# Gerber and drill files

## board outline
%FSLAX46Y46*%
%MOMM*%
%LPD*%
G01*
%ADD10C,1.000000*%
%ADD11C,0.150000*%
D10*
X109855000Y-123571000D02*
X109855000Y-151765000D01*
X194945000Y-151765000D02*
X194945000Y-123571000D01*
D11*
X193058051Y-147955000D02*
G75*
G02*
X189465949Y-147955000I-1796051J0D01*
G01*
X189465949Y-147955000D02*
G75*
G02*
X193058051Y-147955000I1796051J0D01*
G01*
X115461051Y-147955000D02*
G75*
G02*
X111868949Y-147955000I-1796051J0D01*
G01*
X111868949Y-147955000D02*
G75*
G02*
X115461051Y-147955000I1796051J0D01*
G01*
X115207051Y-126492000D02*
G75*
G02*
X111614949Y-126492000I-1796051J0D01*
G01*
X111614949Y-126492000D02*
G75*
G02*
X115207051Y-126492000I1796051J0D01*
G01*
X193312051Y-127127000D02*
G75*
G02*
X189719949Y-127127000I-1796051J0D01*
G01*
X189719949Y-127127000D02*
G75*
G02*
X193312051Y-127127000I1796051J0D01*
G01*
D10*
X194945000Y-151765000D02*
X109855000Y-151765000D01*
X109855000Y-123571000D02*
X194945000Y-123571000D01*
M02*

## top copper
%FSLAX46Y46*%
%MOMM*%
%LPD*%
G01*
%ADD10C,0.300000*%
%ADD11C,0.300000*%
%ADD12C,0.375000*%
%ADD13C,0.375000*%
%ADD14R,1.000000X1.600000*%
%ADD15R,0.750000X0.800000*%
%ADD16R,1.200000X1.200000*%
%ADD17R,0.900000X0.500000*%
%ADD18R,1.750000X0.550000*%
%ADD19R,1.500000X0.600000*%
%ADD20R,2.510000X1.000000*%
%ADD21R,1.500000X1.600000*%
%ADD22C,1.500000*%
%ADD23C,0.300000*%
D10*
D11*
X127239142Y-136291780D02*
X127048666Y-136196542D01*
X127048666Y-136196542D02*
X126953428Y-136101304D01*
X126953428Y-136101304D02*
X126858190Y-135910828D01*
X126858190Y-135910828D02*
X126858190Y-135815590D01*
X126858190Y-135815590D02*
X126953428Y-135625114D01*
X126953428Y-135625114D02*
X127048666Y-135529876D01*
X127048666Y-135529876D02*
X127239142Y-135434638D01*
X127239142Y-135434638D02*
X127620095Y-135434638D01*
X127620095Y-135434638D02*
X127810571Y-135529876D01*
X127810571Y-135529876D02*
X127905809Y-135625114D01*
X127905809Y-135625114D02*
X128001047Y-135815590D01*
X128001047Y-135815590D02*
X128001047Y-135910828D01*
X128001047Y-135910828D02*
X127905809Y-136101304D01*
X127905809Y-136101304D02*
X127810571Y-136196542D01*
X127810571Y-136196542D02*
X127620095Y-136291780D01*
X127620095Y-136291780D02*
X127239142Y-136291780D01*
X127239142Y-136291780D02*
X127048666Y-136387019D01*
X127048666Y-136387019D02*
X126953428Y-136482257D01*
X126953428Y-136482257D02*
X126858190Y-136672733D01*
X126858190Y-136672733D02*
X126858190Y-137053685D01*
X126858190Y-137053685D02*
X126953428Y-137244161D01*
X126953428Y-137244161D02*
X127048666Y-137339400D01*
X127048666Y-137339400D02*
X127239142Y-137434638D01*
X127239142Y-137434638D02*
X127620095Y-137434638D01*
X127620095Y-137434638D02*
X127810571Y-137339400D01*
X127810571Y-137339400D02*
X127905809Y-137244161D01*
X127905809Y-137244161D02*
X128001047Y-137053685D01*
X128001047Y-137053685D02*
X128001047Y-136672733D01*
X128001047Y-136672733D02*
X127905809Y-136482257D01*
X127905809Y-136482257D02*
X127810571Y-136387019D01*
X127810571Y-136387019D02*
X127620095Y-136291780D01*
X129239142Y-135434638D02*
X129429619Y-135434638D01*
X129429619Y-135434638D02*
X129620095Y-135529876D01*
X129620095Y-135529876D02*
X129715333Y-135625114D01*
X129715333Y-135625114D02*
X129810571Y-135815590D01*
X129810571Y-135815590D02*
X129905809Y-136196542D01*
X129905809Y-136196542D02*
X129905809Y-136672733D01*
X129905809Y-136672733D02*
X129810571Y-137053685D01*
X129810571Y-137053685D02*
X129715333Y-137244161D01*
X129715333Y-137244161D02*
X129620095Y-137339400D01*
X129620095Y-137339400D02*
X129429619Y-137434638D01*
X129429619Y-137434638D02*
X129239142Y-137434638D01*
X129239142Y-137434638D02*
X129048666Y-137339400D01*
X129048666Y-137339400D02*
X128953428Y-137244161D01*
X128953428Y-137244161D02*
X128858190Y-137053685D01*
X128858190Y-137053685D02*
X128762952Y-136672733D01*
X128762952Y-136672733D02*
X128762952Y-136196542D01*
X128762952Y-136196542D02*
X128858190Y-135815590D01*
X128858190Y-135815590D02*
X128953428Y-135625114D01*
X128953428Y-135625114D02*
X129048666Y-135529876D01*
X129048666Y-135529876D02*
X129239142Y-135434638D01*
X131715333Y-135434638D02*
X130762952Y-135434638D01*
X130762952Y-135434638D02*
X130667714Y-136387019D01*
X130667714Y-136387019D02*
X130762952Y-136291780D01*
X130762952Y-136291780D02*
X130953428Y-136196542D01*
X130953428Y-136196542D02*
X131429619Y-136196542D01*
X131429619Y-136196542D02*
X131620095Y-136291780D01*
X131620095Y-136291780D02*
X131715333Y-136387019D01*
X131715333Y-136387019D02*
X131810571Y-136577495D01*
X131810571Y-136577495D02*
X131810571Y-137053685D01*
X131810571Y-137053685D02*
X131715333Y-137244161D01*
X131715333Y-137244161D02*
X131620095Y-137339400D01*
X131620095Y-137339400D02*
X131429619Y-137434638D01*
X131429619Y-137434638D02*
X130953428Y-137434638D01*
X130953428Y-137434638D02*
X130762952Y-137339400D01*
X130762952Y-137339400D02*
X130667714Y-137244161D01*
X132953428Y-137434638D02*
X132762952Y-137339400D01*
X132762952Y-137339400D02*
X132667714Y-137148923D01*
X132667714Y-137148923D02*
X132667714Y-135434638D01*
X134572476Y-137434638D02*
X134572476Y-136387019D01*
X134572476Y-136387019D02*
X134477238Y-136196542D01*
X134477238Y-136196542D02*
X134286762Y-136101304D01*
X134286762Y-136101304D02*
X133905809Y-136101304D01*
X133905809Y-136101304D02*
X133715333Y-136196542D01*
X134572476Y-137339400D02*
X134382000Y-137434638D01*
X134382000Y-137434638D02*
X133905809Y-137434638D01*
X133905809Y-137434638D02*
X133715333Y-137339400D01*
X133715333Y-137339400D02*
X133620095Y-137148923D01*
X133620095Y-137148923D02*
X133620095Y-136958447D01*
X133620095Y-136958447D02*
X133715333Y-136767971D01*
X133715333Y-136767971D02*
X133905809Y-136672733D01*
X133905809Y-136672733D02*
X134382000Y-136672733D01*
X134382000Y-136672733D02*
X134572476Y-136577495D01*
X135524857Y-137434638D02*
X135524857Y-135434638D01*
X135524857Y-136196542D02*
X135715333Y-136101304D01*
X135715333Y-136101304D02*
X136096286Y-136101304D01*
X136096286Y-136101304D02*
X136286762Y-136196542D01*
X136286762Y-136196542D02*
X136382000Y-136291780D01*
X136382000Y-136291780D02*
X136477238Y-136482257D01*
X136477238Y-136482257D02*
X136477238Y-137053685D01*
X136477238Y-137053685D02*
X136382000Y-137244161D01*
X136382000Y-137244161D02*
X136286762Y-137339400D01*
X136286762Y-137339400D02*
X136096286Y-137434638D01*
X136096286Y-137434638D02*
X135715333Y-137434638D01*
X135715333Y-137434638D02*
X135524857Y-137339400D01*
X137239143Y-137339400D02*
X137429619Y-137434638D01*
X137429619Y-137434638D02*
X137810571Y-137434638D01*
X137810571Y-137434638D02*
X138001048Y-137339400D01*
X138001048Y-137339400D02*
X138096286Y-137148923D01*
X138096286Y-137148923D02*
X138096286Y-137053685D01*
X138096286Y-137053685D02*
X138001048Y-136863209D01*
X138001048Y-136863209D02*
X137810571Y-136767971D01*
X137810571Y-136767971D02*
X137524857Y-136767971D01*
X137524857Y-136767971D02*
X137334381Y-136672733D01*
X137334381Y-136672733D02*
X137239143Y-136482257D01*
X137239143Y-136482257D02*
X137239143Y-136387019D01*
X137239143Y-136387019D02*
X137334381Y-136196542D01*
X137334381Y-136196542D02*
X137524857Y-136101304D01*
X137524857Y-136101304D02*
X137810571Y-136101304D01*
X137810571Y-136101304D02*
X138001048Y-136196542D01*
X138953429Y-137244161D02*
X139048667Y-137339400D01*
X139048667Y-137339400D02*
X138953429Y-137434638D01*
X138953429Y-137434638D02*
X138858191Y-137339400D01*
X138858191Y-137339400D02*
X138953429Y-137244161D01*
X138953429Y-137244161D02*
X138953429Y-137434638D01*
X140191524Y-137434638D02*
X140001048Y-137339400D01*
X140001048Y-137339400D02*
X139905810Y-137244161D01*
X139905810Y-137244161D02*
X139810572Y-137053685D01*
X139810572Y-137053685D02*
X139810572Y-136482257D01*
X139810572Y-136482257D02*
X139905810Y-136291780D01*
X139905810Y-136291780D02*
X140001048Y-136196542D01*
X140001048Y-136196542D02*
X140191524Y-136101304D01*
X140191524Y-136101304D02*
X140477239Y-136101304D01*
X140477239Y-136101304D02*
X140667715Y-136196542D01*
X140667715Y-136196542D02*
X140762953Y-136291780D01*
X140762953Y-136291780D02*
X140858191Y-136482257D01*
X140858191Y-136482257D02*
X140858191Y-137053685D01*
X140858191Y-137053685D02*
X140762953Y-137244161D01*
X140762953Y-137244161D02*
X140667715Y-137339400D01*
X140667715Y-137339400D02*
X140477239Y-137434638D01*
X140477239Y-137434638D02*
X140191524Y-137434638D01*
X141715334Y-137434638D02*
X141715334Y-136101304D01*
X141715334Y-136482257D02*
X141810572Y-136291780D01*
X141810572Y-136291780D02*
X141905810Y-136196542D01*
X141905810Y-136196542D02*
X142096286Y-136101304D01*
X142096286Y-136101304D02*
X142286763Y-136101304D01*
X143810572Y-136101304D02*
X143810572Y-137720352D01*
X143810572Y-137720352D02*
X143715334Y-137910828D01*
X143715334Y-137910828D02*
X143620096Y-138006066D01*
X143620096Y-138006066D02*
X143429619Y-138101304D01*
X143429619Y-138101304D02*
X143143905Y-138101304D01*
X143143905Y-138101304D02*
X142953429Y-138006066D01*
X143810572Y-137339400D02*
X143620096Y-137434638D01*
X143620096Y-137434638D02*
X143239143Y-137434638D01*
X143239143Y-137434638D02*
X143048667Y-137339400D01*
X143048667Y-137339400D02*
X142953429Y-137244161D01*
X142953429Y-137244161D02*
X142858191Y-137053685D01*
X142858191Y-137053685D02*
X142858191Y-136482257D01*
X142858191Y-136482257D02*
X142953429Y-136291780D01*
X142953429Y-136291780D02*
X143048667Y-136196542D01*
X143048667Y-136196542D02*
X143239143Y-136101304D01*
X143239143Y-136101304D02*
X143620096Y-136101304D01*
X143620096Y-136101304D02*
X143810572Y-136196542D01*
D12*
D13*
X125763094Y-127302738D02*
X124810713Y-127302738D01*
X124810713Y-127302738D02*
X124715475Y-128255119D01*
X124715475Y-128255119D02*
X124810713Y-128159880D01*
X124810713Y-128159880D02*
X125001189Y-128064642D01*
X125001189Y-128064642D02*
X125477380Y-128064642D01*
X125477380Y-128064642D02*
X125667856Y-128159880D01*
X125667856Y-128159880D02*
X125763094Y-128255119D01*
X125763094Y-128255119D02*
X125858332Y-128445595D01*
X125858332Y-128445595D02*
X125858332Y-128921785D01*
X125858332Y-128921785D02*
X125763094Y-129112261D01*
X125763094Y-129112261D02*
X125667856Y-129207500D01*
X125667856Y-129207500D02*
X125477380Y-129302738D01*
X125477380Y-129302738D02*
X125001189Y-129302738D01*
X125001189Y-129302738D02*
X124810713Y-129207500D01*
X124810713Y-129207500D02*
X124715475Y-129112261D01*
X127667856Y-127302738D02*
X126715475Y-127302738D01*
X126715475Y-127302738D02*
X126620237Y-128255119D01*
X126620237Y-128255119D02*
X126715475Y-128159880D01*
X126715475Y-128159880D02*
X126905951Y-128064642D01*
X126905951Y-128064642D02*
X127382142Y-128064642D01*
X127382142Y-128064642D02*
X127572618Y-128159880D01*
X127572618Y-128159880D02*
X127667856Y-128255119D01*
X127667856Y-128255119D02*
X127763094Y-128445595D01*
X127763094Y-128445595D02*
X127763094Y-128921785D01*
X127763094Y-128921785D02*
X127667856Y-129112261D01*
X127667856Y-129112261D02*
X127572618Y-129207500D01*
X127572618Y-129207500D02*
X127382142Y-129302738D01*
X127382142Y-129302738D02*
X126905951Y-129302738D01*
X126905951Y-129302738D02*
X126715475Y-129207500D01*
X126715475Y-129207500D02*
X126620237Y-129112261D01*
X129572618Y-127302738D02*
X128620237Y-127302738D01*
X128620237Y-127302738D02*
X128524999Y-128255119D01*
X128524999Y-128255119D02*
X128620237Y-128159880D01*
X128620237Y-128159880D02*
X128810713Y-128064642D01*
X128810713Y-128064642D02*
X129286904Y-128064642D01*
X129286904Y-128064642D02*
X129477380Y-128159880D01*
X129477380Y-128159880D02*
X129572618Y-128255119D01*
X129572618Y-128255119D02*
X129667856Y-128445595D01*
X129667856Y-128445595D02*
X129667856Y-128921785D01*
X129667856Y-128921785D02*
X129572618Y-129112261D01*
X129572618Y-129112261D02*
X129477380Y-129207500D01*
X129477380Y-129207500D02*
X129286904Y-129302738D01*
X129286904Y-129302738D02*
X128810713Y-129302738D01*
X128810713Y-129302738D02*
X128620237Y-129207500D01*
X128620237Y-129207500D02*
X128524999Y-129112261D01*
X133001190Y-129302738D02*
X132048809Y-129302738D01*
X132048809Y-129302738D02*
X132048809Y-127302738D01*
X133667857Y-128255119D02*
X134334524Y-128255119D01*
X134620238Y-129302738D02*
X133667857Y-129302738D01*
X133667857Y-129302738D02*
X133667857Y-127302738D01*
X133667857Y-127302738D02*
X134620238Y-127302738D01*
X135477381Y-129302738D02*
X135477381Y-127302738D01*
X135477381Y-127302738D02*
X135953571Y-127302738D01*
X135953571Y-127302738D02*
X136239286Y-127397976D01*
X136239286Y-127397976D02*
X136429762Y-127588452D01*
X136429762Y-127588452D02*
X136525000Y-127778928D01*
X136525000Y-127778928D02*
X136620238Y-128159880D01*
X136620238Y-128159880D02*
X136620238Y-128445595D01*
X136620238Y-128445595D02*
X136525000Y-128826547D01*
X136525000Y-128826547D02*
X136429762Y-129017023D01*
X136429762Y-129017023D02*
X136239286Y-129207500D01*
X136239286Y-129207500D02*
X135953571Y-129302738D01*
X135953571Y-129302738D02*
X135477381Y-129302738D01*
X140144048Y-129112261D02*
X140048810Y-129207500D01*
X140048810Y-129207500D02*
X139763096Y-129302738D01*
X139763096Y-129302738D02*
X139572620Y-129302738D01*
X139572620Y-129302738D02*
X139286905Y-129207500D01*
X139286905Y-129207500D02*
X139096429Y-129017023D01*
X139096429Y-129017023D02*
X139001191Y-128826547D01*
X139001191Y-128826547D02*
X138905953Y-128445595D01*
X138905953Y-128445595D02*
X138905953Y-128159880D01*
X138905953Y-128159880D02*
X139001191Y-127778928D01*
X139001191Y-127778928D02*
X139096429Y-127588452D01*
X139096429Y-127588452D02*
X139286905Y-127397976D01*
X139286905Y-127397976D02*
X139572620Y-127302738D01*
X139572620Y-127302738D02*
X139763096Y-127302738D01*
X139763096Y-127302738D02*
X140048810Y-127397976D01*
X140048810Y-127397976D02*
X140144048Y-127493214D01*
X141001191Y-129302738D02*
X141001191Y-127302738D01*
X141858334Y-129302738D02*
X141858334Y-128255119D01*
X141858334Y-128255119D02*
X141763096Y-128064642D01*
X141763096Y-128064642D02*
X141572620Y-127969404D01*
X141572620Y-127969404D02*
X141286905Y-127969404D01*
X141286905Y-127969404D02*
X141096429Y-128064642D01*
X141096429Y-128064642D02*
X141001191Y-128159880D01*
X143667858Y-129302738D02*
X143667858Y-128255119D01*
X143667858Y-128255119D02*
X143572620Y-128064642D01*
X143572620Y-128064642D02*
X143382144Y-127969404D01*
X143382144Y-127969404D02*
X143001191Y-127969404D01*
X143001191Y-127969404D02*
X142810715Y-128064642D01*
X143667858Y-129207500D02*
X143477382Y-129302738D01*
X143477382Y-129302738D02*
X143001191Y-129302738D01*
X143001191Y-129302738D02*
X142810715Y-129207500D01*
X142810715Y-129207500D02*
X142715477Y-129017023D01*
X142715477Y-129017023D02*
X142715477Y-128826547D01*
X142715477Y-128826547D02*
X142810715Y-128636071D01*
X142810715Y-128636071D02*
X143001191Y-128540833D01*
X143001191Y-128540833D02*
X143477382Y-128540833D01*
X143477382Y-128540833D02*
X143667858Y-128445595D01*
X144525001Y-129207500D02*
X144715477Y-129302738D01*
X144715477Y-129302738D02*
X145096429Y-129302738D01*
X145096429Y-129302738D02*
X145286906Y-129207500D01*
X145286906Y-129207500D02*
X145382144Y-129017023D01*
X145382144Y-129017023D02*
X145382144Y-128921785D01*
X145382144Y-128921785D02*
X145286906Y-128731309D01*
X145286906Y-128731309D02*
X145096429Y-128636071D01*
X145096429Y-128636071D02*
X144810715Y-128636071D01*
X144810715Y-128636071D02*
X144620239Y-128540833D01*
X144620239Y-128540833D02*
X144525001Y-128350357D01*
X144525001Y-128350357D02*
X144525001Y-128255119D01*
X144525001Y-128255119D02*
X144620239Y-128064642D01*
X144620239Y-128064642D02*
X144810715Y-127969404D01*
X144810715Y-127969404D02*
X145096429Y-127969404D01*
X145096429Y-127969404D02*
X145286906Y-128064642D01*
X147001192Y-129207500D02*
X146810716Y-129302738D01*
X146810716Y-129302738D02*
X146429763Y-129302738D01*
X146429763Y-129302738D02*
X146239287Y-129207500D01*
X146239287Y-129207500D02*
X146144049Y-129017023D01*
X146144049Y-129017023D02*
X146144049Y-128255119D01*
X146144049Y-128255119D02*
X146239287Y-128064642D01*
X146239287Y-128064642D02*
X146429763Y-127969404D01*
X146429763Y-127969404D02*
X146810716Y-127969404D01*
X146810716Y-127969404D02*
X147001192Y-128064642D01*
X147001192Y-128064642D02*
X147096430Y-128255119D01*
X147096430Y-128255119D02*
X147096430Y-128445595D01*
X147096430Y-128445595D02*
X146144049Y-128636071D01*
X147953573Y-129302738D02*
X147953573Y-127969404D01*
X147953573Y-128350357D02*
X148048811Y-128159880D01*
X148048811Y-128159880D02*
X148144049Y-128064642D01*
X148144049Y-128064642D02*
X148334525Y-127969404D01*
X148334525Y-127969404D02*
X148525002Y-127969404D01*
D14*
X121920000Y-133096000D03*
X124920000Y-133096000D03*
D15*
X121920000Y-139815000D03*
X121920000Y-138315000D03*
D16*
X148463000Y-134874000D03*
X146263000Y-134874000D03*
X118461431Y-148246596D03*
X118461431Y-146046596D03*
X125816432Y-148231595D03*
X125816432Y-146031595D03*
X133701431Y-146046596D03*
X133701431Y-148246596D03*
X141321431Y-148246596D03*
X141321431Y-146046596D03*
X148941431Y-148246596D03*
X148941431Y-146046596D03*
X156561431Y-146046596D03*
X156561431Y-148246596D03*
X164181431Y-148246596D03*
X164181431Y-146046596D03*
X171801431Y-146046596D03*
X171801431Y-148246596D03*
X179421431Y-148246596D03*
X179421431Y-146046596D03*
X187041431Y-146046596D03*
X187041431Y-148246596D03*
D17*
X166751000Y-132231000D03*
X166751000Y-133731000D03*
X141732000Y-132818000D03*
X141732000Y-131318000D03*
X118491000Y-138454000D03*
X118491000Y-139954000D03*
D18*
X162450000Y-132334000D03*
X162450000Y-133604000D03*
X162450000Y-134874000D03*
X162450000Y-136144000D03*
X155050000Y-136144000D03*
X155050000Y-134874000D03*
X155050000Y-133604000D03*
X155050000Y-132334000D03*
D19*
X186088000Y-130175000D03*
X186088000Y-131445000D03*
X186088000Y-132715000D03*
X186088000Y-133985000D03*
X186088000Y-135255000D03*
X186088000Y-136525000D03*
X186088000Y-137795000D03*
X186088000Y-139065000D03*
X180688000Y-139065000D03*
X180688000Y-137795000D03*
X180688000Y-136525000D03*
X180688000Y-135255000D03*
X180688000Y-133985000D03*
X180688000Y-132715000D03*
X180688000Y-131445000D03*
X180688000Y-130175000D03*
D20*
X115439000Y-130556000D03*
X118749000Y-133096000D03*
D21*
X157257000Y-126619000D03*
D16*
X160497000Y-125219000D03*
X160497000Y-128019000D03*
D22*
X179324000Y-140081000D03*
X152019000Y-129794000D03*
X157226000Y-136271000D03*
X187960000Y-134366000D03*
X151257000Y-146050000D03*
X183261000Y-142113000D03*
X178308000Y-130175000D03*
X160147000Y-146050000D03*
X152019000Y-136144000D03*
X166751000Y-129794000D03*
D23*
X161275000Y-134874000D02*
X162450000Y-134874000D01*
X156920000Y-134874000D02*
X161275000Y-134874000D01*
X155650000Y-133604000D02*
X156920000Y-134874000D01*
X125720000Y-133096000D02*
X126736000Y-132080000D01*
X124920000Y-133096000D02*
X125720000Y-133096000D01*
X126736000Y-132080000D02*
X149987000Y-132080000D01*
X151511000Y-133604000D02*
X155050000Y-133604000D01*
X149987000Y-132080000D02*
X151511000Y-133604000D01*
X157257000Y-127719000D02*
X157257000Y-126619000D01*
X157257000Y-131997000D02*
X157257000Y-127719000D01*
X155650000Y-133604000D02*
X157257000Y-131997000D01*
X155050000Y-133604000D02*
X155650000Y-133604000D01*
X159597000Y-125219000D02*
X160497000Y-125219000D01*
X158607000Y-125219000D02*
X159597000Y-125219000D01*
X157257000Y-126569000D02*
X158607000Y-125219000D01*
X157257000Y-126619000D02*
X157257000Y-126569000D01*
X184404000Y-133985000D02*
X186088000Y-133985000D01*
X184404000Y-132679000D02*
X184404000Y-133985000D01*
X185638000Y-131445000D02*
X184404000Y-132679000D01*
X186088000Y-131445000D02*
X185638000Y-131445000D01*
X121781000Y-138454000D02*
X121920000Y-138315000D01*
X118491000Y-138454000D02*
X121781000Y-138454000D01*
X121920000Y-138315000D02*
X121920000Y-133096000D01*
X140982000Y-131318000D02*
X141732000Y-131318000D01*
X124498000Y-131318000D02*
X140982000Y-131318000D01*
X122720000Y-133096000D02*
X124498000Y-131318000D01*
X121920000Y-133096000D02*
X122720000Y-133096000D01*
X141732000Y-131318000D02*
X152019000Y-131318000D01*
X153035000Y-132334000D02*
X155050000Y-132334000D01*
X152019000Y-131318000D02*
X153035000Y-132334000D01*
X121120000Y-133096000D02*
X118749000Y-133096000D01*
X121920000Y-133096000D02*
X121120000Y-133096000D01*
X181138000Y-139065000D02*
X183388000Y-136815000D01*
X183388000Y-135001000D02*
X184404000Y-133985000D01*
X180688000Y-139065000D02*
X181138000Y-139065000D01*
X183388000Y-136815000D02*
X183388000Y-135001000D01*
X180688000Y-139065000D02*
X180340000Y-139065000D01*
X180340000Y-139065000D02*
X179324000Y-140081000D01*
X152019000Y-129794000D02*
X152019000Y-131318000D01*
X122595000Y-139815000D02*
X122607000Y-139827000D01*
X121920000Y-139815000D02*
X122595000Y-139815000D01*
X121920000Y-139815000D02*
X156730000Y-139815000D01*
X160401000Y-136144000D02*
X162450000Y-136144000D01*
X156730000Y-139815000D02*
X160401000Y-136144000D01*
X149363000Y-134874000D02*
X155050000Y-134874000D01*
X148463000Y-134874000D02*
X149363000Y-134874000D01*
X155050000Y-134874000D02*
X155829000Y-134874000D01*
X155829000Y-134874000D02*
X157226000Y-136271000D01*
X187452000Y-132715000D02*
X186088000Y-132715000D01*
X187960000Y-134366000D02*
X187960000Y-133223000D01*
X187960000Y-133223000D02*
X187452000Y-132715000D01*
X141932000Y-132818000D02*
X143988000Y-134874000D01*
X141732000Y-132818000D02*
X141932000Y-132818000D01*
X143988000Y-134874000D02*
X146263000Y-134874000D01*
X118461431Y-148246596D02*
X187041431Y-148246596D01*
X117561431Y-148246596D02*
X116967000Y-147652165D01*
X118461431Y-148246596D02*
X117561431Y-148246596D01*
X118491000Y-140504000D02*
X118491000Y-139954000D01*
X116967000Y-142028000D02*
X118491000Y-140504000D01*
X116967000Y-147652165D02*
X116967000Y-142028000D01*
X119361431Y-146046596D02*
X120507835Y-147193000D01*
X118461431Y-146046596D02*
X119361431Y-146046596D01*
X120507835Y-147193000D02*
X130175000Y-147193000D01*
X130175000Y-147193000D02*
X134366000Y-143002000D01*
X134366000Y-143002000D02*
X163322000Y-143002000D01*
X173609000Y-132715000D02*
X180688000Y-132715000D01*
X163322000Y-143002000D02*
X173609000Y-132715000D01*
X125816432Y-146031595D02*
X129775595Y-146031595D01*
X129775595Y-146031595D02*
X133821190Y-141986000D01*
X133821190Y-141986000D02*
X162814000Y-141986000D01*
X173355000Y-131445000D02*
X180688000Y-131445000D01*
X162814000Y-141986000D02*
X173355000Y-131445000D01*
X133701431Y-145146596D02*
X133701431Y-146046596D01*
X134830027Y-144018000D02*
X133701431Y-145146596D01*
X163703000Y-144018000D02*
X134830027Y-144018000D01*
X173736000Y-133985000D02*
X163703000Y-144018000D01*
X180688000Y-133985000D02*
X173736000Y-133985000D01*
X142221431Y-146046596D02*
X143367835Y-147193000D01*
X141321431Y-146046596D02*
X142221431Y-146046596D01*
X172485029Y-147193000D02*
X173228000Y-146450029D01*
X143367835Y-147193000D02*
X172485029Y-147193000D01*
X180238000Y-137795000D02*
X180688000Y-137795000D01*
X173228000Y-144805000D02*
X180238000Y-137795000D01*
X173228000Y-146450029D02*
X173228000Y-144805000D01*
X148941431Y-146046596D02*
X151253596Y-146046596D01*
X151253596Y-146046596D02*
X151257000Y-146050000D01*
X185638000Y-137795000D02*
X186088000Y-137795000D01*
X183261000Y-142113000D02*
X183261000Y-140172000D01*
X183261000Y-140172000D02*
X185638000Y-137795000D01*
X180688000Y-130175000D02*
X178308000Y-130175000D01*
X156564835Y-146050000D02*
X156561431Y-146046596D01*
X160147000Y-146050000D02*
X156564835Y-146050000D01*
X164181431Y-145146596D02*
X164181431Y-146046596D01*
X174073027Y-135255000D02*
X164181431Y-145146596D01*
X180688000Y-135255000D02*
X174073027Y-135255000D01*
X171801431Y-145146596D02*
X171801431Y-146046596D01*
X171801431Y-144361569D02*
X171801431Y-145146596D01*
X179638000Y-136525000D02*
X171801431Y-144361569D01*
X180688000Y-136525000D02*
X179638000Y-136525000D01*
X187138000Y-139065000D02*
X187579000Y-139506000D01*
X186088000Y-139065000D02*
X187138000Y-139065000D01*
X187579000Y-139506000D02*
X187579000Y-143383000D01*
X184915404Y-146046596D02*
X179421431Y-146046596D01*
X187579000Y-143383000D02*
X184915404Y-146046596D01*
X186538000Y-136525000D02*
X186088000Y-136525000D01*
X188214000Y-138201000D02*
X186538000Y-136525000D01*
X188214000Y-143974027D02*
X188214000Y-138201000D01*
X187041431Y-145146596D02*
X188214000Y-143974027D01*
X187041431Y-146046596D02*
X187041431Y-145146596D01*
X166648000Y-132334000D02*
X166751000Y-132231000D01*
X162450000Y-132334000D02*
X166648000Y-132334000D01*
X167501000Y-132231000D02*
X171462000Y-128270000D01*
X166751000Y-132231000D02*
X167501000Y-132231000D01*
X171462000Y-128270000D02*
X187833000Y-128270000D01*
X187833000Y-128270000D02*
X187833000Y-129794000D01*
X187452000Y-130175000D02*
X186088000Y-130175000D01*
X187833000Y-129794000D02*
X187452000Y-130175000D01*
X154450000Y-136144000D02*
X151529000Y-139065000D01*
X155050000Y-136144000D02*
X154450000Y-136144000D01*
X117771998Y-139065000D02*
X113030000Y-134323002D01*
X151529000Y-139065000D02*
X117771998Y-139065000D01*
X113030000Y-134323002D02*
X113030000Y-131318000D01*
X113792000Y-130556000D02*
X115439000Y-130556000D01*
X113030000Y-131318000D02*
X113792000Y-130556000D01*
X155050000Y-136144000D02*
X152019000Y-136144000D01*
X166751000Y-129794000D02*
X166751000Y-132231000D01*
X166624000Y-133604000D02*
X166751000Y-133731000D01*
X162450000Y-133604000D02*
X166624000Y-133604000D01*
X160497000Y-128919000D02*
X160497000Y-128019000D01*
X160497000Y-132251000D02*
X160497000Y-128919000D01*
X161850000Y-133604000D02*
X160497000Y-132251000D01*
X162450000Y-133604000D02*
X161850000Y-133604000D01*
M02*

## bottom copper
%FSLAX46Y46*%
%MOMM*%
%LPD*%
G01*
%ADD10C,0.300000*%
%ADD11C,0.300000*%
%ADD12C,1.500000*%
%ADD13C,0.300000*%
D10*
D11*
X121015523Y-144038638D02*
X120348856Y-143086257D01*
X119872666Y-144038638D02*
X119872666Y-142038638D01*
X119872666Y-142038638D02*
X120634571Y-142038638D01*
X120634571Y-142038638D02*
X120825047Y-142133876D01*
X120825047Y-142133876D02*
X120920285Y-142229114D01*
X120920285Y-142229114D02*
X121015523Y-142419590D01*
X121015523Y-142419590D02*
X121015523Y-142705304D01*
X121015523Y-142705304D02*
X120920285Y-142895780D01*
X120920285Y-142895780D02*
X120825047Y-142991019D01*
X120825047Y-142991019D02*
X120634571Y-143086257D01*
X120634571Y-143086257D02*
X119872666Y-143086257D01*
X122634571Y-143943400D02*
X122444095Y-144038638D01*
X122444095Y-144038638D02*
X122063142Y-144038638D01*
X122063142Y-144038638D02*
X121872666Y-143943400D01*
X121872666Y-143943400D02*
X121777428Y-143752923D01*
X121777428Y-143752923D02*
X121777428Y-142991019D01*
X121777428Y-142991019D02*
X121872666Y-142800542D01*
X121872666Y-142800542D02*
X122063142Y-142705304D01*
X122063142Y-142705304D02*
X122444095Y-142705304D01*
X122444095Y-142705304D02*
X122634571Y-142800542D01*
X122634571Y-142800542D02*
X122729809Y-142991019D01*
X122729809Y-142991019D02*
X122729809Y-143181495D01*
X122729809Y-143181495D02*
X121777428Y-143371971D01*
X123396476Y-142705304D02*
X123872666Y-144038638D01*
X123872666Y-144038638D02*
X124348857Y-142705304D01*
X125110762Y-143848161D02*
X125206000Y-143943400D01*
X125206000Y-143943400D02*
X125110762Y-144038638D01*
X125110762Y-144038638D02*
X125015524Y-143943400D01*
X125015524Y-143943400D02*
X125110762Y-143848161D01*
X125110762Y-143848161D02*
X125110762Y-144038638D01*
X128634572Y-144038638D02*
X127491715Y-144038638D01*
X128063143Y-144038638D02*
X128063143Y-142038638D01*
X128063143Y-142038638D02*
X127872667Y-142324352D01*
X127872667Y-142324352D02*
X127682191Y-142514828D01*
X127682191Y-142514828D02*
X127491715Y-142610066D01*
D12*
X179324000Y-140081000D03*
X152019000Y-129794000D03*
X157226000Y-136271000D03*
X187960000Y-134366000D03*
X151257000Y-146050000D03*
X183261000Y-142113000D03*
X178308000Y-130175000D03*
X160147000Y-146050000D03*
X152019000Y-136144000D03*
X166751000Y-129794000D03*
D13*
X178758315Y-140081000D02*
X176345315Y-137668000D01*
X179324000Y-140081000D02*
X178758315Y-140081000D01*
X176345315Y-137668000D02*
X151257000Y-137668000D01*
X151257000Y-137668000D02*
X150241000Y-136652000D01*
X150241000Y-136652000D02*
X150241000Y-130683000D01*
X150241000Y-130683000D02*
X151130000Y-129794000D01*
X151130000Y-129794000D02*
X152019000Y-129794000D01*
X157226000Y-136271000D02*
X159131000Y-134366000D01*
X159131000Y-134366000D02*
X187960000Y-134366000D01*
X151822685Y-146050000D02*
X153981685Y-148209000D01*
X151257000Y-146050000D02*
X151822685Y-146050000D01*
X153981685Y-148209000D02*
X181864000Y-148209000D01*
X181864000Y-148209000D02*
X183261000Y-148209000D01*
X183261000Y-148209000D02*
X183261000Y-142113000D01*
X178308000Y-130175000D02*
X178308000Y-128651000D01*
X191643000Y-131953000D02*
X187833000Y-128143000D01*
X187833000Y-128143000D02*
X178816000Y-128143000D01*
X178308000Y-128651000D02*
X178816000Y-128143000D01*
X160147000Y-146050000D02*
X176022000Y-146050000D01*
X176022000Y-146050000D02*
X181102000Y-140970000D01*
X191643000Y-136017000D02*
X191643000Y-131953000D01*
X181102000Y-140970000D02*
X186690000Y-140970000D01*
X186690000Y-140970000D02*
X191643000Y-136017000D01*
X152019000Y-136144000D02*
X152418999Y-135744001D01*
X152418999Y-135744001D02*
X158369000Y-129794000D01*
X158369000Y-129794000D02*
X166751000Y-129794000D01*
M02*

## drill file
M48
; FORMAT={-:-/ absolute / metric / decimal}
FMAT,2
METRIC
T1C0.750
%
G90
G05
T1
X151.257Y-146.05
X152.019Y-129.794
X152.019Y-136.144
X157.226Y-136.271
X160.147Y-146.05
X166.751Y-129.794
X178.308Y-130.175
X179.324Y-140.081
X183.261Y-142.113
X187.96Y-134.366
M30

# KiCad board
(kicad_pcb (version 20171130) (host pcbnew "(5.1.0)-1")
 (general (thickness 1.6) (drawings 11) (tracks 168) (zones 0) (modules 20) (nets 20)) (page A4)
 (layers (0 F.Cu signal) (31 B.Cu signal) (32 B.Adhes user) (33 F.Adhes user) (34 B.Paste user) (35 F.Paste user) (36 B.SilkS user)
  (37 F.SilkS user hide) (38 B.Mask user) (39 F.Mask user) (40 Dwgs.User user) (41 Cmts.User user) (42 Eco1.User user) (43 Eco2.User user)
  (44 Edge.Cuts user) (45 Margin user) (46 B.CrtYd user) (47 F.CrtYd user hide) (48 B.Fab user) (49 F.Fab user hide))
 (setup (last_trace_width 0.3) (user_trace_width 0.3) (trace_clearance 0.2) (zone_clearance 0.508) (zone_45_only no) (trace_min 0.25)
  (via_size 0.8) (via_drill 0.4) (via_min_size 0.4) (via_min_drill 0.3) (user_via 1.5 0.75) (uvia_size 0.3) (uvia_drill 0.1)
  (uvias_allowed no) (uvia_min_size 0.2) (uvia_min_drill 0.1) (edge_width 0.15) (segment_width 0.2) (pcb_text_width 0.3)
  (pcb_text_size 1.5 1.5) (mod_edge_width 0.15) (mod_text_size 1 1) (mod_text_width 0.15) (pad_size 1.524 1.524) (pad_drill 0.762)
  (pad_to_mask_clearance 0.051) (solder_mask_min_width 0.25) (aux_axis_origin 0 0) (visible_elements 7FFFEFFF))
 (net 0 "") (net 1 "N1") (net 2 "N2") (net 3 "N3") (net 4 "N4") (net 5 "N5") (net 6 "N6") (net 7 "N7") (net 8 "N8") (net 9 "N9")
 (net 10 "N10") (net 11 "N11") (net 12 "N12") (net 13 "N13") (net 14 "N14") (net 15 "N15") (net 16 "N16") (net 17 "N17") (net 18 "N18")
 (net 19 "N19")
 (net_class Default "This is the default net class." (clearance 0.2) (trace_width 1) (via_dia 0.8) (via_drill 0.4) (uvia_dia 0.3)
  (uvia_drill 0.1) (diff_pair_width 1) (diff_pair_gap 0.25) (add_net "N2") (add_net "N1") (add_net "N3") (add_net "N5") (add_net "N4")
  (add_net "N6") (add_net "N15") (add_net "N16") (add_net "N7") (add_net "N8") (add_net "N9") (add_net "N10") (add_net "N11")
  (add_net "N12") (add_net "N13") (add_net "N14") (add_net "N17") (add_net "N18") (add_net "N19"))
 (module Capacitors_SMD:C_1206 (layer F.Cu) (at 123.42 133.096 180)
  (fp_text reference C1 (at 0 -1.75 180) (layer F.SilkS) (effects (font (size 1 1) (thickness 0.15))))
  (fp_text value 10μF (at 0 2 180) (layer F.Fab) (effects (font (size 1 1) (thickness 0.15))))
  (pad 2 smd rect (at 1.5 0 180) (size 1 1.6) (layers F.Cu F.Paste F.Mask) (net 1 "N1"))
  (pad 1 smd rect (at -1.5 0 180) (size 1 1.6) (layers F.Cu F.Paste F.Mask) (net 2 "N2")))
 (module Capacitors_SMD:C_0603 (layer F.Cu) (at 121.92 139.065 90)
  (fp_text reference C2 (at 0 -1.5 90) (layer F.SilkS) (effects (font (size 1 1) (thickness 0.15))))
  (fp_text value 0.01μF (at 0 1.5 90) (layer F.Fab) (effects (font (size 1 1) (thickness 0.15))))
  (pad 1 smd rect (at -0.75 0 90) (size 0.8 0.75) (layers F.Cu F.Paste F.Mask) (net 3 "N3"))
  (pad 2 smd rect (at 0.75 0 90) (size 0.8 0.75) (layers F.Cu F.Paste F.Mask) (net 1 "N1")))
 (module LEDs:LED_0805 (layer F.Cu) (at 147.363 134.874)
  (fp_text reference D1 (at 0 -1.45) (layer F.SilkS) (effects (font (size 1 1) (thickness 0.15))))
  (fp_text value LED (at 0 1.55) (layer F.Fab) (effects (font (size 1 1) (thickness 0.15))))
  (pad 2 smd rect (at 1.1 0 180) (size 1.2 1.2) (layers F.Cu F.Paste F.Mask) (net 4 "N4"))
  (pad 1 smd rect (at -1.1 0 180) (size 1.2 1.2) (layers F.Cu F.Paste F.Mask) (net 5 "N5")))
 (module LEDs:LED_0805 (layer F.Cu) (at 118.461431 147.146596 90)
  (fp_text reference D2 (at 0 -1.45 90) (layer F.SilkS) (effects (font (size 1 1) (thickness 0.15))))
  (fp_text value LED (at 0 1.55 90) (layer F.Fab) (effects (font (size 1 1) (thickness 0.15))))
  (pad 1 smd rect (at -1.1 0 270) (size 1.2 1.2) (layers F.Cu F.Paste F.Mask) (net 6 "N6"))
  (pad 2 smd rect (at 1.1 0 270) (size 1.2 1.2) (layers F.Cu F.Paste F.Mask) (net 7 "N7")))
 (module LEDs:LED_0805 (layer F.Cu) (at 125.816432 147.131595 90)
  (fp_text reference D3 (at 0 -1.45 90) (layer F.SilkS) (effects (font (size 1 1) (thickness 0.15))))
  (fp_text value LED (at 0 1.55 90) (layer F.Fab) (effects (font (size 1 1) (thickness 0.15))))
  (pad 1 smd rect (at -1.1 0 270) (size 1.2 1.2) (layers F.Cu F.Paste F.Mask) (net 6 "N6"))
  (pad 2 smd rect (at 1.1 0 270) (size 1.2 1.2) (layers F.Cu F.Paste F.Mask) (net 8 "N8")))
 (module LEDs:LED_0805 (layer F.Cu) (at 133.701431 147.146596 90)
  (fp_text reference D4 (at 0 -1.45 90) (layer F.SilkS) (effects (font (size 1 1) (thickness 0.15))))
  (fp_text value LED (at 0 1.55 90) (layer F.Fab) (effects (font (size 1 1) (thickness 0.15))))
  (pad 2 smd rect (at 1.1 0 270) (size 1.2 1.2) (layers F.Cu F.Paste F.Mask) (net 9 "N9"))
  (pad 1 smd rect (at -1.1 0 270) (size 1.2 1.2) (layers F.Cu F.Paste F.Mask) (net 6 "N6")))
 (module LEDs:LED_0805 (layer F.Cu) (at 141.321431 147.146596 90)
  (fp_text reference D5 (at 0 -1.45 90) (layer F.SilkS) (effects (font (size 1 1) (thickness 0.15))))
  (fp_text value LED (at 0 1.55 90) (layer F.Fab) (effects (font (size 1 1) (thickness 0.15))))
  (pad 1 smd rect (at -1.1 0 270) (size 1.2 1.2) (layers F.Cu F.Paste F.Mask) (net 6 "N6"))
  (pad 2 smd rect (at 1.1 0 270) (size 1.2 1.2) (layers F.Cu F.Paste F.Mask) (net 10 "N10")))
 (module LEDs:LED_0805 (layer F.Cu) (at 148.941431 147.146596 90)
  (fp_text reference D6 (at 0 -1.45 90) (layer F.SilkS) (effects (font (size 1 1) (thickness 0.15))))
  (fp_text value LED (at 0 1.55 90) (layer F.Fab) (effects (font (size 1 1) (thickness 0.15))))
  (pad 1 smd rect (at -1.1 0 270) (size 1.2 1.2) (layers F.Cu F.Paste F.Mask) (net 6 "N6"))
  (pad 2 smd rect (at 1.1 0 270) (size 1.2 1.2) (layers F.Cu F.Paste F.Mask) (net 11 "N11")))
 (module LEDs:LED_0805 (layer F.Cu) (at 156.561431 147.146596 90)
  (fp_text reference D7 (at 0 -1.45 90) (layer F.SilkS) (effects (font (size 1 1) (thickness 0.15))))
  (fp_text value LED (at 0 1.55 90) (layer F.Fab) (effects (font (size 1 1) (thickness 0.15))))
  (pad 2 smd rect (at 1.1 0 270) (size 1.2 1.2) (layers F.Cu F.Paste F.Mask) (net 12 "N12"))
  (pad 1 smd rect (at -1.1 0 270) (size 1.2 1.2) (layers F.Cu F.Paste F.Mask) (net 6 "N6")))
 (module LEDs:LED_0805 (layer F.Cu) (at 164.181431 147.146596 90)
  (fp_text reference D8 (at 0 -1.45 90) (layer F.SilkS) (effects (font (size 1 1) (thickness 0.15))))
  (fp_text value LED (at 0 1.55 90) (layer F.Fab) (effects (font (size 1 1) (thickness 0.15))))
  (pad 1 smd rect (at -1.1 0 270) (size 1.2 1.2) (layers F.Cu F.Paste F.Mask) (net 6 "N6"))
  (pad 2 smd rect (at 1.1 0 270) (size 1.2 1.2) (layers F.Cu F.Paste F.Mask) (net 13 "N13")))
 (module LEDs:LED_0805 (layer F.Cu) (at 171.801431 147.146596 90)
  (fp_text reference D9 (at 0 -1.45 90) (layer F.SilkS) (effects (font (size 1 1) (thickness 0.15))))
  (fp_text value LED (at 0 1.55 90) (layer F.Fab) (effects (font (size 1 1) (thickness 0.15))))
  (pad 2 smd rect (at 1.1 0 270) (size 1.2 1.2) (layers F.Cu F.Paste F.Mask) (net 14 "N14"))
  (pad 1 smd rect (at -1.1 0 270) (size 1.2 1.2) (layers F.Cu F.Paste F.Mask) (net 6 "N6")))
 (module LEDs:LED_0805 (layer F.Cu) (at 179.421431 147.146596 90)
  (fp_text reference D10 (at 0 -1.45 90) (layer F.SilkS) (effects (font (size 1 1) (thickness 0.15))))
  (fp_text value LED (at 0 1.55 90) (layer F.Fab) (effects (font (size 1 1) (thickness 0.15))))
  (pad 1 smd rect (at -1.1 0 270) (size 1.2 1.2) (layers F.Cu F.Paste F.Mask) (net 6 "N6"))
  (pad 2 smd rect (at 1.1 0 270) (size 1.2 1.2) (layers F.Cu F.Paste F.Mask) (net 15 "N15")))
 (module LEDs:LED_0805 (layer F.Cu) (at 187.041431 147.146596 90)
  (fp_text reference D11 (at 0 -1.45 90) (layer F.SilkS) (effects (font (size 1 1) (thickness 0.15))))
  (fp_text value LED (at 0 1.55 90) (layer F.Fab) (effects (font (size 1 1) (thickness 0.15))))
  (pad 2 smd rect (at 1.1 0 270) (size 1.2 1.2) (layers F.Cu F.Paste F.Mask) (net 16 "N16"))
  (pad 1 smd rect (at -1.1 0 270) (size 1.2 1.2) (layers F.Cu F.Paste F.Mask) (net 6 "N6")))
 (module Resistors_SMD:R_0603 (layer F.Cu) (at 166.751 132.981 270)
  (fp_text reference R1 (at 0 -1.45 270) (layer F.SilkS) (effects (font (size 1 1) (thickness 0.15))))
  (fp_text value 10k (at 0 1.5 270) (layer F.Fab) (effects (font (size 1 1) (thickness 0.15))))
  (pad 1 smd rect (at -0.75 0 270) (size 0.5 0.9) (layers F.Cu F.Paste F.Mask) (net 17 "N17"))
  (pad 2 smd rect (at 0.75 0 270) (size 0.5 0.9) (layers F.Cu F.Paste F.Mask) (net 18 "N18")))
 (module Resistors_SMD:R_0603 (layer F.Cu) (at 141.732 132.068 90)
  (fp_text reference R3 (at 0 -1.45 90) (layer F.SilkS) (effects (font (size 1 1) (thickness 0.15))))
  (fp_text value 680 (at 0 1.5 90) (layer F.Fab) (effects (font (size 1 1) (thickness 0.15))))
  (pad 1 smd rect (at -0.75 0 90) (size 0.5 0.9) (layers F.Cu F.Paste F.Mask) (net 5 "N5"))
  (pad 2 smd rect (at 0.75 0 90) (size 0.5 0.9) (layers F.Cu F.Paste F.Mask) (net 1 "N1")))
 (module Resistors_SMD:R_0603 (layer F.Cu) (at 118.491 139.204 90)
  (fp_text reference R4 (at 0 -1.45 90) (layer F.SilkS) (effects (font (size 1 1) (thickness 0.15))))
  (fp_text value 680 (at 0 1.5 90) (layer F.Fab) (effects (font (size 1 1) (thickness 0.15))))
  (pad 2 smd rect (at 0.75 0 90) (size 0.5 0.9) (layers F.Cu F.Paste F.Mask) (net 1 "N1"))
  (pad 1 smd rect (at -0.75 0 90) (size 0.5 0.9) (layers F.Cu F.Paste F.Mask) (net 6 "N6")))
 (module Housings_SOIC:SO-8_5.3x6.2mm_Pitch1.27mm (layer F.Cu) (at 158.75 134.239)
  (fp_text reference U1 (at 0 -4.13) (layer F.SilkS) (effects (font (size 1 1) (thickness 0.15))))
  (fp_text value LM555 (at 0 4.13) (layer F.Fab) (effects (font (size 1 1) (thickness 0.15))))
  (pad 8 smd rect (at 3.7 -1.905) (size 1.75 0.55) (layers F.Cu F.Paste F.Mask) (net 17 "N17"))
  (pad 7 smd rect (at 3.7 -0.635) (size 1.75 0.55) (layers F.Cu F.Paste F.Mask) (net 18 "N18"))
  (pad 6 smd rect (at 3.7 0.635) (size 1.75 0.55) (layers F.Cu F.Paste F.Mask) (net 2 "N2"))
  (pad 5 smd rect (at 3.7 1.905) (size 1.75 0.55) (layers F.Cu F.Paste F.Mask) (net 3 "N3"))
  (pad 4 smd rect (at -3.7 1.905) (size 1.75 0.55) (layers F.Cu F.Paste F.Mask) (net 17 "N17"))
  (pad 3 smd rect (at -3.7 0.635) (size 1.75 0.55) (layers F.Cu F.Paste F.Mask) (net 4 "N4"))
  (pad 2 smd rect (at -3.7 -0.635) (size 1.75 0.55) (layers F.Cu F.Paste F.Mask) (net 2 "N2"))
  (pad 1 smd rect (at -3.7 -1.905) (size 1.75 0.55) (layers F.Cu F.Paste F.Mask) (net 1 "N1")))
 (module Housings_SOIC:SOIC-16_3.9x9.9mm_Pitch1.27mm (layer F.Cu) (at 183.388 134.62)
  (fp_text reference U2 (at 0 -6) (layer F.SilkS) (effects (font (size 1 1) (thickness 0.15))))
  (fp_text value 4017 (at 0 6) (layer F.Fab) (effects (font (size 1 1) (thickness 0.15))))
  (pad 16 smd rect (at 2.7 -4.445) (size 1.5 0.6) (layers F.Cu F.Paste F.Mask) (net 17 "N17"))
  (pad 15 smd rect (at 2.7 -3.175) (size 1.5 0.6) (layers F.Cu F.Paste F.Mask) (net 1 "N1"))
  (pad 14 smd rect (at 2.7 -1.905) (size 1.5 0.6) (layers F.Cu F.Paste F.Mask) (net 4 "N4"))
  (pad 13 smd rect (at 2.7 -0.635) (size 1.5 0.6) (layers F.Cu F.Paste F.Mask) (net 1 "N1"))
  (pad 12 smd rect (at 2.7 0.635) (size 1.5 0.6) (layers F.Cu F.Paste F.Mask) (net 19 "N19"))
  (pad 11 smd rect (at 2.7 1.905) (size 1.5 0.6) (layers F.Cu F.Paste F.Mask) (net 16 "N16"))
  (pad 10 smd rect (at 2.7 3.175) (size 1.5 0.6) (layers F.Cu F.Paste F.Mask) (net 11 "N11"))
  (pad 9 smd rect (at 2.7 4.445) (size 1.5 0.6) (layers F.Cu F.Paste F.Mask) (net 15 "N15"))
  (pad 8 smd rect (at -2.7 4.445) (size 1.5 0.6) (layers F.Cu F.Paste F.Mask) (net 1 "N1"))
  (pad 7 smd rect (at -2.7 3.175) (size 1.5 0.6) (layers F.Cu F.Paste F.Mask) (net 10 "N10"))
  (pad 6 smd rect (at -2.7 1.905) (size 1.5 0.6) (layers F.Cu F.Paste F.Mask) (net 14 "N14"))
  (pad 5 smd rect (at -2.7 0.635) (size 1.5 0.6) (layers F.Cu F.Paste F.Mask) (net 13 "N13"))
  (pad 4 smd rect (at -2.7 -0.635) (size 1.5 0.6) (layers F.Cu F.Paste F.Mask) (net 9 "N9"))
  (pad 3 smd rect (at -2.7 -1.905) (size 1.5 0.6) (layers F.Cu F.Paste F.Mask) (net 7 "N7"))
  (pad 2 smd rect (at -2.7 -3.175) (size 1.5 0.6) (layers F.Cu F.Paste F.Mask) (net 8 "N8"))
  (pad 1 smd rect (at -2.7 -4.445) (size 1.5 0.6) (layers F.Cu F.Paste F.Mask) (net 12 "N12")))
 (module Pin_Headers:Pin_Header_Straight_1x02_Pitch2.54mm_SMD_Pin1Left (layer F.Cu) (at 117.094 131.826 180)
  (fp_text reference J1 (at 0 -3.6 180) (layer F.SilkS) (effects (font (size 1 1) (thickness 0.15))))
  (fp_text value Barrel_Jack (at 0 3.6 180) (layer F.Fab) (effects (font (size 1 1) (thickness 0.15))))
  (pad 2 smd rect (at 1.655 1.27 180) (size 2.51 1) (layers F.Cu F.Paste F.Mask) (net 17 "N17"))
  (pad 1 smd rect (at -1.655 -1.27 180) (size 2.51 1) (layers F.Cu F.Paste F.Mask) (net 1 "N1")))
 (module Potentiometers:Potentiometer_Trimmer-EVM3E (layer F.Cu) (at 158.877 126.619 90)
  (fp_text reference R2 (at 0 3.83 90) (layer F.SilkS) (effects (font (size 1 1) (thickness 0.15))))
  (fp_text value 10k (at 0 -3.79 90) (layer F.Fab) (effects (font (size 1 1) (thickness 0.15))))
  (pad 2 smd rect (at 0 -1.62 90) (size 1.6 1.5) (layers F.Cu F.Paste F.Mask) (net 2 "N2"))
  (pad 3 smd rect (at 1.4 1.62 90) (size 1.2 1.2) (layers F.Cu F.Paste F.Mask) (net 2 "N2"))
  (pad 1 smd rect (at -1.4 1.62 90) (size 1.2 1.2) (layers F.Cu F.Paste F.Mask) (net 18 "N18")))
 (gr_line (start 109.855 123.571) (end 109.855 151.765) (layer Edge.Cuts) (width 1))
 (gr_line (start 194.945 151.765) (end 194.945 123.571) (layer Edge.Cuts) (width 1))
 (gr_circle (center 191.262 147.955) (end 193.058051 147.955) (layer Edge.Cuts) (width 0.15))
 (gr_circle (center 113.665 147.955) (end 115.461051 147.955) (layer Edge.Cuts) (width 0.15))
 (gr_circle (center 113.411 126.492) (end 115.207051 126.492) (layer Edge.Cuts) (width 0.15))
 (gr_circle (center 191.516 127.127) (end 193.312051 127.127) (layer Edge.Cuts) (width 0.15))
 (gr_line (start 194.945 151.765) (end 109.855 151.765) (layer Edge.Cuts) (width 1))
 (gr_line (start 109.855 123.571) (end 194.945 123.571) (layer Edge.Cuts) (width 1))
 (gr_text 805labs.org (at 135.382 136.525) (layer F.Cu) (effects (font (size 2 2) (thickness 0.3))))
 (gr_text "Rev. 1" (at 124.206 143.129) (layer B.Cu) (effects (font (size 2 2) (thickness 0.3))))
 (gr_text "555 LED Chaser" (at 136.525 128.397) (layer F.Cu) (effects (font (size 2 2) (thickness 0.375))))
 (segment (start 161.275 134.874) (end 162.45 134.874) (width 0.3) (layer F.Cu) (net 2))
 (segment (start 156.92 134.874) (end 161.275 134.874) (width 0.3) (layer F.Cu) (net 2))
 (segment (start 155.65 133.604) (end 156.92 134.874) (width 0.3) (layer F.Cu) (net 2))
 (segment (start 125.72 133.096) (end 126.736 132.08) (width 0.3) (layer F.Cu) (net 2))
 (segment (start 124.92 133.096) (end 125.72 133.096) (width 0.3) (layer F.Cu) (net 2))
 (segment (start 126.736 132.08) (end 149.987 132.08) (width 0.3) (layer F.Cu) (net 2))
 (segment (start 151.511 133.604) (end 155.05 133.604) (width 0.3) (layer F.Cu) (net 2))
 (segment (start 149.987 132.08) (end 151.511 133.604) (width 0.3) (layer F.Cu) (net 2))
 (segment (start 157.257 127.719) (end 157.257 126.619) (width 0.3) (layer F.Cu) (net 2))
 (segment (start 157.257 131.997) (end 157.257 127.719) (width 0.3) (layer F.Cu) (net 2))
 (segment (start 155.65 133.604) (end 157.257 131.997) (width 0.3) (layer F.Cu) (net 2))
 (segment (start 155.05 133.604) (end 155.65 133.604) (width 0.3) (layer F.Cu) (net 2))
 (segment (start 159.597 125.219) (end 160.497 125.219) (width 0.3) (layer F.Cu) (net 2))
 (segment (start 158.607 125.219) (end 159.597 125.219) (width 0.3) (layer F.Cu) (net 2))
 (segment (start 157.257 126.569) (end 158.607 125.219) (width 0.3) (layer F.Cu) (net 2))
 (segment (start 157.257 126.619) (end 157.257 126.569) (width 0.3) (layer F.Cu) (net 2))
 (segment (start 184.404 133.985) (end 186.088 133.985) (width 0.3) (layer F.Cu) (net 1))
 (segment (start 184.404 132.679) (end 184.404 133.985) (width 0.3) (layer F.Cu) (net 1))
 (segment (start 185.638 131.445) (end 184.404 132.679) (width 0.3) (layer F.Cu) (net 1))
 (segment (start 186.088 131.445) (end 185.638 131.445) (width 0.3) (layer F.Cu) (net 1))
 (segment (start 121.781 138.454) (end 121.92 138.315) (width 0.3) (layer F.Cu) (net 1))
 (segment (start 118.491 138.454) (end 121.781 138.454) (width 0.3) (layer F.Cu) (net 1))
 (segment (start 121.92 138.315) (end 121.92 133.096) (width 0.3) (layer F.Cu) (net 1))
 (segment (start 140.982 131.318) (end 141.732 131.318) (width 0.3) (layer F.Cu) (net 1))
 (segment (start 124.498 131.318) (end 140.982 131.318) (width 0.3) (layer F.Cu) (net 1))
 (segment (start 122.72 133.096) (end 124.498 131.318) (width 0.3) (layer F.Cu) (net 1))
 (segment (start 121.92 133.096) (end 122.72 133.096) (width 0.3) (layer F.Cu) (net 1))
 (segment (start 141.732 131.318) (end 152.019 131.318) (width 0.3) (layer F.Cu) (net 1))
 (segment (start 153.035 132.334) (end 155.05 132.334) (width 0.3) (layer F.Cu) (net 1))
 (segment (start 152.019 131.318) (end 153.035 132.334) (width 0.3) (layer F.Cu) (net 1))
 (segment (start 121.12 133.096) (end 118.749 133.096) (width 0.3) (layer F.Cu) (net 1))
 (segment (start 121.92 133.096) (end 121.12 133.096) (width 0.3) (layer F.Cu) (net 1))
 (segment (start 181.138 139.065) (end 183.388 136.815) (width 0.3) (layer F.Cu) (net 1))
 (segment (start 183.388 135.001) (end 184.404 133.985) (width 0.3) (layer F.Cu) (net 1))
 (segment (start 180.688 139.065) (end 181.138 139.065) (width 0.3) (layer F.Cu) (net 1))
 (segment (start 183.388 136.815) (end 183.388 135.001) (width 0.3) (layer F.Cu) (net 1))
 (via (at 179.324 140.081) (size 1.5) (drill 0.75) (layers F.Cu B.Cu) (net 1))
 (segment (start 180.688 139.065) (end 180.34 139.065) (width 0.3) (layer F.Cu) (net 1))
 (segment (start 180.34 139.065) (end 179.324 140.081) (width 0.3) (layer F.Cu) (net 1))
 (segment (start 178.758315 140.081) (end 176.345315 137.668) (width 0.3) (layer B.Cu) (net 1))
 (segment (start 179.324 140.081) (end 178.758315 140.081) (width 0.3) (layer B.Cu) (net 1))
 (segment (start 176.345315 137.668) (end 151.257 137.668) (width 0.3) (layer B.Cu) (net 1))
 (segment (start 151.257 137.668) (end 150.241 136.652) (width 0.3) (layer B.Cu) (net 1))
 (segment (start 150.241 136.652) (end 150.241 130.683) (width 0.3) (layer B.Cu) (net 1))
 (via (at 152.019 129.794) (size 1.5) (drill 0.75) (layers F.Cu B.Cu) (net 1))
 (segment (start 150.241 130.683) (end 151.13 129.794) (width 0.3) (layer B.Cu) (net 1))
 (segment (start 151.13 129.794) (end 152.019 129.794) (width 0.3) (layer B.Cu) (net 1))
 (segment (start 152.019 129.794) (end 152.019 131.318) (width 0.3) (layer F.Cu) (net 1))
 (segment (start 122.595 139.815) (end 122.607 139.827) (width 0.3) (layer F.Cu) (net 3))
 (segment (start 121.92 139.815) (end 122.595 139.815) (width 0.3) (layer F.Cu) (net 3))
 (segment (start 121.92 139.815) (end 156.73 139.815) (width 0.3) (layer F.Cu) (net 3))
 (segment (start 160.401 136.144) (end 162.45 136.144) (width 0.3) (layer F.Cu) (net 3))
 (segment (start 156.73 139.815) (end 160.401 136.144) (width 0.3) (layer F.Cu) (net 3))
 (segment (start 149.363 134.874) (end 155.05 134.874) (width 0.3) (layer F.Cu) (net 4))
 (segment (start 148.463 134.874) (end 149.363 134.874) (width 0.3) (layer F.Cu) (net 4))
 (via (at 157.226 136.271) (size 1.5) (drill 0.75) (layers F.Cu B.Cu) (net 4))
 (segment (start 155.05 134.874) (end 155.829 134.874) (width 0.3) (layer F.Cu) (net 4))
 (segment (start 155.829 134.874) (end 157.226 136.271) (width 0.3) (layer F.Cu) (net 4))
 (via (at 187.96 134.366) (size 1.5) (drill 0.75) (layers F.Cu B.Cu) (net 4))
 (segment (start 157.226 136.271) (end 159.131 134.366) (width 0.3) (layer B.Cu) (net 4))
 (segment (start 159.131 134.366) (end 187.96 134.366) (width 0.3) (layer B.Cu) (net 4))
 (segment (start 187.452 132.715) (end 186.088 132.715) (width 0.3) (layer F.Cu) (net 4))
 (segment (start 187.96 134.366) (end 187.96 133.223) (width 0.3) (layer F.Cu) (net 4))
 (segment (start 187.96 133.223) (end 187.452 132.715) (width 0.3) (layer F.Cu) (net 4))
 (segment (start 141.932 132.818) (end 143.988 134.874) (width 0.3) (layer F.Cu) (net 5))
 (segment (start 141.732 132.818) (end 141.932 132.818) (width 0.3) (layer F.Cu) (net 5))
 (segment (start 143.988 134.874) (end 146.263 134.874) (width 0.3) (layer F.Cu) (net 5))
 (segment (start 118.461431 148.246596) (end 187.041431 148.246596) (width 0.3) (layer F.Cu) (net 6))
 (segment (start 117.561431 148.246596) (end 116.967 147.652165) (width 0.3) (layer F.Cu) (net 6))
 (segment (start 118.461431 148.246596) (end 117.561431 148.246596) (width 0.3) (layer F.Cu) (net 6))
 (segment (start 118.491 140.504) (end 118.491 139.954) (width 0.3) (layer F.Cu) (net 6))
 (segment (start 116.967 142.028) (end 118.491 140.504) (width 0.3) (layer F.Cu) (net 6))
 (segment (start 116.967 147.652165) (end 116.967 142.028) (width 0.3) (layer F.Cu) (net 6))
 (segment (start 119.361431 146.046596) (end 120.507835 147.193) (width 0.3) (layer F.Cu) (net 7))
 (segment (start 118.461431 146.046596) (end 119.361431 146.046596) (width 0.3) (layer F.Cu) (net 7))
 (segment (start 120.507835 147.193) (end 130.175 147.193) (width 0.3) (layer F.Cu) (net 7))
 (segment (start 130.175 147.193) (end 134.366 143.002) (width 0.3) (layer F.Cu) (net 7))
 (segment (start 134.366 143.002) (end 163.322 143.002) (width 0.3) (layer F.Cu) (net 7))
 (segment (start 173.609 132.715) (end 180.688 132.715) (width 0.3) (layer F.Cu) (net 7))
 (segment (start 163.322 143.002) (end 173.609 132.715) (width 0.3) (layer F.Cu) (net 7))
 (segment (start 125.816432 146.031595) (end 129.775595 146.031595) (width 0.3) (layer F.Cu) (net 8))
 (segment (start 129.775595 146.031595) (end 133.82119 141.986) (width 0.3) (layer F.Cu) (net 8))
 (segment (start 133.82119 141.986) (end 162.814 141.986) (width 0.3) (layer F.Cu) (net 8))
 (segment (start 173.355 131.445) (end 180.688 131.445) (width 0.3) (layer F.Cu) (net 8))
 (segment (start 162.814 141.986) (end 173.355 131.445) (width 0.3) (layer F.Cu) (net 8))
 (segment (start 133.701431 145.146596) (end 133.701431 146.046596) (width 0.3) (layer F.Cu) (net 9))
 (segment (start 134.830027 144.018) (end 133.701431 145.146596) (width 0.3) (layer F.Cu) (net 9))
 (segment (start 163.703 144.018) (end 134.830027 144.018) (width 0.3) (layer F.Cu) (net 9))
 (segment (start 173.736 133.985) (end 163.703 144.018) (width 0.3) (layer F.Cu) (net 9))
 (segment (start 180.688 133.985) (end 173.736 133.985) (width 0.3) (layer F.Cu) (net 9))
 (segment (start 142.221431 146.046596) (end 143.367835 147.193) (width 0.3) (layer F.Cu) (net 10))
 (segment (start 141.321431 146.046596) (end 142.221431 146.046596) (width 0.3) (layer F.Cu) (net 10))
 (segment (start 172.485029 147.193) (end 173.228 146.450029) (width 0.3) (layer F.Cu) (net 10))
 (segment (start 143.367835 147.193) (end 172.485029 147.193) (width 0.3) (layer F.Cu) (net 10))
 (segment (start 180.238 137.795) (end 180.688 137.795) (width 0.3) (layer F.Cu) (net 10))
 (segment (start 173.228 144.805) (end 180.238 137.795) (width 0.3) (layer F.Cu) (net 10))
 (segment (start 173.228 146.450029) (end 173.228 144.805) (width 0.3) (layer F.Cu) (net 10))
 (via (at 151.257 146.05) (size 1.5) (drill 0.75) (layers F.Cu B.Cu) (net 11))
 (segment (start 148.941431 146.046596) (end 151.253596 146.046596) (width 0.3) (layer F.Cu) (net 11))
 (segment (start 151.253596 146.046596) (end 151.257 146.05) (width 0.3) (layer F.Cu) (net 11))
 (segment (start 151.822685 146.05) (end 153.981685 148.209) (width 0.3) (layer B.Cu) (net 11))
 (segment (start 151.257 146.05) (end 151.822685 146.05) (width 0.3) (layer B.Cu) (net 11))
 (segment (start 153.981685 148.209) (end 181.864 148.209) (width 0.3) (layer B.Cu) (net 11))
 (segment (start 181.864 148.209) (end 183.261 148.209) (width 0.3) (layer B.Cu) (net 11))
 (via (at 183.261 142.113) (size 1.5) (drill 0.75) (layers F.Cu B.Cu) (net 11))
 (segment (start 183.261 148.209) (end 183.261 142.113) (width 0.3) (layer B.Cu) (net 11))
 (segment (start 185.638 137.795) (end 186.088 137.795) (width 0.3) (layer F.Cu) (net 11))
 (segment (start 183.261 142.113) (end 183.261 140.172) (width 0.3) (layer F.Cu) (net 11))
 (segment (start 183.261 140.172) (end 185.638 137.795) (width 0.3) (layer F.Cu) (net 11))
 (via (at 178.308 130.175) (size 1.5) (drill 0.75) (layers F.Cu B.Cu) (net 12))
 (segment (start 180.688 130.175) (end 178.308 130.175) (width 0.3) (layer F.Cu) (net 12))
 (segment (start 178.308 130.175) (end 178.308 128.651) (width 0.3) (layer B.Cu) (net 12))
 (segment (start 156.564835 146.05) (end 156.561431 146.046596) (width 0.3) (layer F.Cu) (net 12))
 (segment (start 160.147 146.05) (end 156.564835 146.05) (width 0.3) (layer F.Cu) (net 12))
 (via (at 160.147 146.05) (size 1.5) (drill 0.75) (layers F.Cu B.Cu) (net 12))
 (segment (start 191.643 131.953) (end 187.833 128.143) (width 0.3) (layer B.Cu) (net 12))
 (segment (start 187.833 128.143) (end 178.816 128.143) (width 0.3) (layer B.Cu) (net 12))
 (segment (start 178.308 128.651) (end 178.816 128.143) (width 0.3) (layer B.Cu) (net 12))
 (segment (start 160.147 146.05) (end 176.022 146.05) (width 0.3) (layer B.Cu) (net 12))
 (segment (start 176.022 146.05) (end 181.102 140.97) (width 0.3) (layer B.Cu) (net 12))
 (segment (start 191.643 136.017) (end 191.643 131.953) (width 0.3) (layer B.Cu) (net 12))
 (segment (start 181.102 140.97) (end 186.69 140.97) (width 0.3) (layer B.Cu) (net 12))
 (segment (start 186.69 140.97) (end 191.643 136.017) (width 0.3) (layer B.Cu) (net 12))
 (segment (start 164.181431 145.146596) (end 164.181431 146.046596) (width 0.3) (layer F.Cu) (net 13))
 (segment (start 174.073027 135.255) (end 164.181431 145.146596) (width 0.3) (layer F.Cu) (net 13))
 (segment (start 180.688 135.255) (end 174.073027 135.255) (width 0.3) (layer F.Cu) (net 13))
 (segment (start 171.801431 145.146596) (end 171.801431 146.046596) (width 0.3) (layer F.Cu) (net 14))
 (segment (start 171.801431 144.361569) (end 171.801431 145.146596) (width 0.3) (layer F.Cu) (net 14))
 (segment (start 179.638 136.525) (end 171.801431 144.361569) (width 0.3) (layer F.Cu) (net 14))
 (segment (start 180.688 136.525) (end 179.638 136.525) (width 0.3) (layer F.Cu) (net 14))
 (segment (start 187.138 139.065) (end 187.579 139.506) (width 0.3) (layer F.Cu) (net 15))
 (segment (start 186.088 139.065) (end 187.138 139.065) (width 0.3) (layer F.Cu) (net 15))
 (segment (start 187.579 139.506) (end 187.579 143.383) (width 0.3) (layer F.Cu) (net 15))
 (segment (start 184.915404 146.046596) (end 179.421431 146.046596) (width 0.3) (layer F.Cu) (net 15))
 (segment (start 187.579 143.383) (end 184.915404 146.046596) (width 0.3) (layer F.Cu) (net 15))
 (segment (start 186.538 136.525) (end 186.088 136.525) (width 0.3) (layer F.Cu) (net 16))
 (segment (start 188.214 138.201) (end 186.538 136.525) (width 0.3) (layer F.Cu) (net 16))
 (segment (start 188.214 143.974027) (end 188.214 138.201) (width 0.3) (layer F.Cu) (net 16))
 (segment (start 187.041431 145.146596) (end 188.214 143.974027) (width 0.3) (layer F.Cu) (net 16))
 (segment (start 187.041431 146.046596) (end 187.041431 145.146596) (width 0.3) (layer F.Cu) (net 16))
 (segment (start 166.648 132.334) (end 166.751 132.231) (width 0.3) (layer F.Cu) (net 17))
 (segment (start 162.45 132.334) (end 166.648 132.334) (width 0.3) (layer F.Cu) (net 17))
 (segment (start 167.501 132.231) (end 171.462 128.27) (width 0.3) (layer F.Cu) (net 17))
 (segment (start 166.751 132.231) (end 167.501 132.231) (width 0.3) (layer F.Cu) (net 17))
 (segment (start 171.462 128.27) (end 187.833 128.27) (width 0.3) (layer F.Cu) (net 17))
 (segment (start 187.833 128.27) (end 187.833 129.794) (width 0.3) (layer F.Cu) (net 17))
 (segment (start 187.452 130.175) (end 186.088 130.175) (width 0.3) (layer F.Cu) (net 17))
 (segment (start 187.833 129.794) (end 187.452 130.175) (width 0.3) (layer F.Cu) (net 17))
 (segment (start 154.45 136.144) (end 151.529 139.065) (width 0.3) (layer F.Cu) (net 17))
 (segment (start 155.05 136.144) (end 154.45 136.144) (width 0.3) (layer F.Cu) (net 17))
 (segment (start 117.771998 139.065) (end 113.03 134.323002) (width 0.3) (layer F.Cu) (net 17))
 (segment (start 151.529 139.065) (end 117.771998 139.065) (width 0.3) (layer F.Cu) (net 17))
 (segment (start 113.03 134.323002) (end 113.03 131.318) (width 0.3) (layer F.Cu) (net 17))
 (segment (start 113.792 130.556) (end 115.439 130.556) (width 0.3) (layer F.Cu) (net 17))
 (segment (start 113.03 131.318) (end 113.792 130.556) (width 0.3) (layer F.Cu) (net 17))
 (via (at 152.019 136.144) (size 1.5) (drill 0.75) (layers F.Cu B.Cu) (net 17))
 (segment (start 155.05 136.144) (end 152.019 136.144) (width 0.3) (layer F.Cu) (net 17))
 (segment (start 152.019 136.144) (end 152.418999 135.744001) (width 0.3) (layer B.Cu) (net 17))
 (via (at 166.751 129.794) (size 1.5) (drill 0.75) (layers F.Cu B.Cu) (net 17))
 (segment (start 152.418999 135.744001) (end 158.369 129.794) (width 0.3) (layer B.Cu) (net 17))
 (segment (start 158.369 129.794) (end 166.751 129.794) (width 0.3) (layer B.Cu) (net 17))
 (segment (start 166.751 129.794) (end 166.751 132.231) (width 0.3) (layer F.Cu) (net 17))
 (segment (start 166.624 133.604) (end 166.751 133.731) (width 0.3) (layer F.Cu) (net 18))
 (segment (start 162.45 133.604) (end 166.624 133.604) (width 0.3) (layer F.Cu) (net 18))
 (segment (start 160.497 128.919) (end 160.497 128.019) (width 0.3) (layer F.Cu) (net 18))
 (segment (start 160.497 132.251) (end 160.497 128.919) (width 0.3) (layer F.Cu) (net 18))
 (segment (start 161.85 133.604) (end 160.497 132.251) (width 0.3) (layer F.Cu) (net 18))
 (segment (start 162.45 133.604) (end 161.85 133.604) (width 0.3) (layer F.Cu) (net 18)))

